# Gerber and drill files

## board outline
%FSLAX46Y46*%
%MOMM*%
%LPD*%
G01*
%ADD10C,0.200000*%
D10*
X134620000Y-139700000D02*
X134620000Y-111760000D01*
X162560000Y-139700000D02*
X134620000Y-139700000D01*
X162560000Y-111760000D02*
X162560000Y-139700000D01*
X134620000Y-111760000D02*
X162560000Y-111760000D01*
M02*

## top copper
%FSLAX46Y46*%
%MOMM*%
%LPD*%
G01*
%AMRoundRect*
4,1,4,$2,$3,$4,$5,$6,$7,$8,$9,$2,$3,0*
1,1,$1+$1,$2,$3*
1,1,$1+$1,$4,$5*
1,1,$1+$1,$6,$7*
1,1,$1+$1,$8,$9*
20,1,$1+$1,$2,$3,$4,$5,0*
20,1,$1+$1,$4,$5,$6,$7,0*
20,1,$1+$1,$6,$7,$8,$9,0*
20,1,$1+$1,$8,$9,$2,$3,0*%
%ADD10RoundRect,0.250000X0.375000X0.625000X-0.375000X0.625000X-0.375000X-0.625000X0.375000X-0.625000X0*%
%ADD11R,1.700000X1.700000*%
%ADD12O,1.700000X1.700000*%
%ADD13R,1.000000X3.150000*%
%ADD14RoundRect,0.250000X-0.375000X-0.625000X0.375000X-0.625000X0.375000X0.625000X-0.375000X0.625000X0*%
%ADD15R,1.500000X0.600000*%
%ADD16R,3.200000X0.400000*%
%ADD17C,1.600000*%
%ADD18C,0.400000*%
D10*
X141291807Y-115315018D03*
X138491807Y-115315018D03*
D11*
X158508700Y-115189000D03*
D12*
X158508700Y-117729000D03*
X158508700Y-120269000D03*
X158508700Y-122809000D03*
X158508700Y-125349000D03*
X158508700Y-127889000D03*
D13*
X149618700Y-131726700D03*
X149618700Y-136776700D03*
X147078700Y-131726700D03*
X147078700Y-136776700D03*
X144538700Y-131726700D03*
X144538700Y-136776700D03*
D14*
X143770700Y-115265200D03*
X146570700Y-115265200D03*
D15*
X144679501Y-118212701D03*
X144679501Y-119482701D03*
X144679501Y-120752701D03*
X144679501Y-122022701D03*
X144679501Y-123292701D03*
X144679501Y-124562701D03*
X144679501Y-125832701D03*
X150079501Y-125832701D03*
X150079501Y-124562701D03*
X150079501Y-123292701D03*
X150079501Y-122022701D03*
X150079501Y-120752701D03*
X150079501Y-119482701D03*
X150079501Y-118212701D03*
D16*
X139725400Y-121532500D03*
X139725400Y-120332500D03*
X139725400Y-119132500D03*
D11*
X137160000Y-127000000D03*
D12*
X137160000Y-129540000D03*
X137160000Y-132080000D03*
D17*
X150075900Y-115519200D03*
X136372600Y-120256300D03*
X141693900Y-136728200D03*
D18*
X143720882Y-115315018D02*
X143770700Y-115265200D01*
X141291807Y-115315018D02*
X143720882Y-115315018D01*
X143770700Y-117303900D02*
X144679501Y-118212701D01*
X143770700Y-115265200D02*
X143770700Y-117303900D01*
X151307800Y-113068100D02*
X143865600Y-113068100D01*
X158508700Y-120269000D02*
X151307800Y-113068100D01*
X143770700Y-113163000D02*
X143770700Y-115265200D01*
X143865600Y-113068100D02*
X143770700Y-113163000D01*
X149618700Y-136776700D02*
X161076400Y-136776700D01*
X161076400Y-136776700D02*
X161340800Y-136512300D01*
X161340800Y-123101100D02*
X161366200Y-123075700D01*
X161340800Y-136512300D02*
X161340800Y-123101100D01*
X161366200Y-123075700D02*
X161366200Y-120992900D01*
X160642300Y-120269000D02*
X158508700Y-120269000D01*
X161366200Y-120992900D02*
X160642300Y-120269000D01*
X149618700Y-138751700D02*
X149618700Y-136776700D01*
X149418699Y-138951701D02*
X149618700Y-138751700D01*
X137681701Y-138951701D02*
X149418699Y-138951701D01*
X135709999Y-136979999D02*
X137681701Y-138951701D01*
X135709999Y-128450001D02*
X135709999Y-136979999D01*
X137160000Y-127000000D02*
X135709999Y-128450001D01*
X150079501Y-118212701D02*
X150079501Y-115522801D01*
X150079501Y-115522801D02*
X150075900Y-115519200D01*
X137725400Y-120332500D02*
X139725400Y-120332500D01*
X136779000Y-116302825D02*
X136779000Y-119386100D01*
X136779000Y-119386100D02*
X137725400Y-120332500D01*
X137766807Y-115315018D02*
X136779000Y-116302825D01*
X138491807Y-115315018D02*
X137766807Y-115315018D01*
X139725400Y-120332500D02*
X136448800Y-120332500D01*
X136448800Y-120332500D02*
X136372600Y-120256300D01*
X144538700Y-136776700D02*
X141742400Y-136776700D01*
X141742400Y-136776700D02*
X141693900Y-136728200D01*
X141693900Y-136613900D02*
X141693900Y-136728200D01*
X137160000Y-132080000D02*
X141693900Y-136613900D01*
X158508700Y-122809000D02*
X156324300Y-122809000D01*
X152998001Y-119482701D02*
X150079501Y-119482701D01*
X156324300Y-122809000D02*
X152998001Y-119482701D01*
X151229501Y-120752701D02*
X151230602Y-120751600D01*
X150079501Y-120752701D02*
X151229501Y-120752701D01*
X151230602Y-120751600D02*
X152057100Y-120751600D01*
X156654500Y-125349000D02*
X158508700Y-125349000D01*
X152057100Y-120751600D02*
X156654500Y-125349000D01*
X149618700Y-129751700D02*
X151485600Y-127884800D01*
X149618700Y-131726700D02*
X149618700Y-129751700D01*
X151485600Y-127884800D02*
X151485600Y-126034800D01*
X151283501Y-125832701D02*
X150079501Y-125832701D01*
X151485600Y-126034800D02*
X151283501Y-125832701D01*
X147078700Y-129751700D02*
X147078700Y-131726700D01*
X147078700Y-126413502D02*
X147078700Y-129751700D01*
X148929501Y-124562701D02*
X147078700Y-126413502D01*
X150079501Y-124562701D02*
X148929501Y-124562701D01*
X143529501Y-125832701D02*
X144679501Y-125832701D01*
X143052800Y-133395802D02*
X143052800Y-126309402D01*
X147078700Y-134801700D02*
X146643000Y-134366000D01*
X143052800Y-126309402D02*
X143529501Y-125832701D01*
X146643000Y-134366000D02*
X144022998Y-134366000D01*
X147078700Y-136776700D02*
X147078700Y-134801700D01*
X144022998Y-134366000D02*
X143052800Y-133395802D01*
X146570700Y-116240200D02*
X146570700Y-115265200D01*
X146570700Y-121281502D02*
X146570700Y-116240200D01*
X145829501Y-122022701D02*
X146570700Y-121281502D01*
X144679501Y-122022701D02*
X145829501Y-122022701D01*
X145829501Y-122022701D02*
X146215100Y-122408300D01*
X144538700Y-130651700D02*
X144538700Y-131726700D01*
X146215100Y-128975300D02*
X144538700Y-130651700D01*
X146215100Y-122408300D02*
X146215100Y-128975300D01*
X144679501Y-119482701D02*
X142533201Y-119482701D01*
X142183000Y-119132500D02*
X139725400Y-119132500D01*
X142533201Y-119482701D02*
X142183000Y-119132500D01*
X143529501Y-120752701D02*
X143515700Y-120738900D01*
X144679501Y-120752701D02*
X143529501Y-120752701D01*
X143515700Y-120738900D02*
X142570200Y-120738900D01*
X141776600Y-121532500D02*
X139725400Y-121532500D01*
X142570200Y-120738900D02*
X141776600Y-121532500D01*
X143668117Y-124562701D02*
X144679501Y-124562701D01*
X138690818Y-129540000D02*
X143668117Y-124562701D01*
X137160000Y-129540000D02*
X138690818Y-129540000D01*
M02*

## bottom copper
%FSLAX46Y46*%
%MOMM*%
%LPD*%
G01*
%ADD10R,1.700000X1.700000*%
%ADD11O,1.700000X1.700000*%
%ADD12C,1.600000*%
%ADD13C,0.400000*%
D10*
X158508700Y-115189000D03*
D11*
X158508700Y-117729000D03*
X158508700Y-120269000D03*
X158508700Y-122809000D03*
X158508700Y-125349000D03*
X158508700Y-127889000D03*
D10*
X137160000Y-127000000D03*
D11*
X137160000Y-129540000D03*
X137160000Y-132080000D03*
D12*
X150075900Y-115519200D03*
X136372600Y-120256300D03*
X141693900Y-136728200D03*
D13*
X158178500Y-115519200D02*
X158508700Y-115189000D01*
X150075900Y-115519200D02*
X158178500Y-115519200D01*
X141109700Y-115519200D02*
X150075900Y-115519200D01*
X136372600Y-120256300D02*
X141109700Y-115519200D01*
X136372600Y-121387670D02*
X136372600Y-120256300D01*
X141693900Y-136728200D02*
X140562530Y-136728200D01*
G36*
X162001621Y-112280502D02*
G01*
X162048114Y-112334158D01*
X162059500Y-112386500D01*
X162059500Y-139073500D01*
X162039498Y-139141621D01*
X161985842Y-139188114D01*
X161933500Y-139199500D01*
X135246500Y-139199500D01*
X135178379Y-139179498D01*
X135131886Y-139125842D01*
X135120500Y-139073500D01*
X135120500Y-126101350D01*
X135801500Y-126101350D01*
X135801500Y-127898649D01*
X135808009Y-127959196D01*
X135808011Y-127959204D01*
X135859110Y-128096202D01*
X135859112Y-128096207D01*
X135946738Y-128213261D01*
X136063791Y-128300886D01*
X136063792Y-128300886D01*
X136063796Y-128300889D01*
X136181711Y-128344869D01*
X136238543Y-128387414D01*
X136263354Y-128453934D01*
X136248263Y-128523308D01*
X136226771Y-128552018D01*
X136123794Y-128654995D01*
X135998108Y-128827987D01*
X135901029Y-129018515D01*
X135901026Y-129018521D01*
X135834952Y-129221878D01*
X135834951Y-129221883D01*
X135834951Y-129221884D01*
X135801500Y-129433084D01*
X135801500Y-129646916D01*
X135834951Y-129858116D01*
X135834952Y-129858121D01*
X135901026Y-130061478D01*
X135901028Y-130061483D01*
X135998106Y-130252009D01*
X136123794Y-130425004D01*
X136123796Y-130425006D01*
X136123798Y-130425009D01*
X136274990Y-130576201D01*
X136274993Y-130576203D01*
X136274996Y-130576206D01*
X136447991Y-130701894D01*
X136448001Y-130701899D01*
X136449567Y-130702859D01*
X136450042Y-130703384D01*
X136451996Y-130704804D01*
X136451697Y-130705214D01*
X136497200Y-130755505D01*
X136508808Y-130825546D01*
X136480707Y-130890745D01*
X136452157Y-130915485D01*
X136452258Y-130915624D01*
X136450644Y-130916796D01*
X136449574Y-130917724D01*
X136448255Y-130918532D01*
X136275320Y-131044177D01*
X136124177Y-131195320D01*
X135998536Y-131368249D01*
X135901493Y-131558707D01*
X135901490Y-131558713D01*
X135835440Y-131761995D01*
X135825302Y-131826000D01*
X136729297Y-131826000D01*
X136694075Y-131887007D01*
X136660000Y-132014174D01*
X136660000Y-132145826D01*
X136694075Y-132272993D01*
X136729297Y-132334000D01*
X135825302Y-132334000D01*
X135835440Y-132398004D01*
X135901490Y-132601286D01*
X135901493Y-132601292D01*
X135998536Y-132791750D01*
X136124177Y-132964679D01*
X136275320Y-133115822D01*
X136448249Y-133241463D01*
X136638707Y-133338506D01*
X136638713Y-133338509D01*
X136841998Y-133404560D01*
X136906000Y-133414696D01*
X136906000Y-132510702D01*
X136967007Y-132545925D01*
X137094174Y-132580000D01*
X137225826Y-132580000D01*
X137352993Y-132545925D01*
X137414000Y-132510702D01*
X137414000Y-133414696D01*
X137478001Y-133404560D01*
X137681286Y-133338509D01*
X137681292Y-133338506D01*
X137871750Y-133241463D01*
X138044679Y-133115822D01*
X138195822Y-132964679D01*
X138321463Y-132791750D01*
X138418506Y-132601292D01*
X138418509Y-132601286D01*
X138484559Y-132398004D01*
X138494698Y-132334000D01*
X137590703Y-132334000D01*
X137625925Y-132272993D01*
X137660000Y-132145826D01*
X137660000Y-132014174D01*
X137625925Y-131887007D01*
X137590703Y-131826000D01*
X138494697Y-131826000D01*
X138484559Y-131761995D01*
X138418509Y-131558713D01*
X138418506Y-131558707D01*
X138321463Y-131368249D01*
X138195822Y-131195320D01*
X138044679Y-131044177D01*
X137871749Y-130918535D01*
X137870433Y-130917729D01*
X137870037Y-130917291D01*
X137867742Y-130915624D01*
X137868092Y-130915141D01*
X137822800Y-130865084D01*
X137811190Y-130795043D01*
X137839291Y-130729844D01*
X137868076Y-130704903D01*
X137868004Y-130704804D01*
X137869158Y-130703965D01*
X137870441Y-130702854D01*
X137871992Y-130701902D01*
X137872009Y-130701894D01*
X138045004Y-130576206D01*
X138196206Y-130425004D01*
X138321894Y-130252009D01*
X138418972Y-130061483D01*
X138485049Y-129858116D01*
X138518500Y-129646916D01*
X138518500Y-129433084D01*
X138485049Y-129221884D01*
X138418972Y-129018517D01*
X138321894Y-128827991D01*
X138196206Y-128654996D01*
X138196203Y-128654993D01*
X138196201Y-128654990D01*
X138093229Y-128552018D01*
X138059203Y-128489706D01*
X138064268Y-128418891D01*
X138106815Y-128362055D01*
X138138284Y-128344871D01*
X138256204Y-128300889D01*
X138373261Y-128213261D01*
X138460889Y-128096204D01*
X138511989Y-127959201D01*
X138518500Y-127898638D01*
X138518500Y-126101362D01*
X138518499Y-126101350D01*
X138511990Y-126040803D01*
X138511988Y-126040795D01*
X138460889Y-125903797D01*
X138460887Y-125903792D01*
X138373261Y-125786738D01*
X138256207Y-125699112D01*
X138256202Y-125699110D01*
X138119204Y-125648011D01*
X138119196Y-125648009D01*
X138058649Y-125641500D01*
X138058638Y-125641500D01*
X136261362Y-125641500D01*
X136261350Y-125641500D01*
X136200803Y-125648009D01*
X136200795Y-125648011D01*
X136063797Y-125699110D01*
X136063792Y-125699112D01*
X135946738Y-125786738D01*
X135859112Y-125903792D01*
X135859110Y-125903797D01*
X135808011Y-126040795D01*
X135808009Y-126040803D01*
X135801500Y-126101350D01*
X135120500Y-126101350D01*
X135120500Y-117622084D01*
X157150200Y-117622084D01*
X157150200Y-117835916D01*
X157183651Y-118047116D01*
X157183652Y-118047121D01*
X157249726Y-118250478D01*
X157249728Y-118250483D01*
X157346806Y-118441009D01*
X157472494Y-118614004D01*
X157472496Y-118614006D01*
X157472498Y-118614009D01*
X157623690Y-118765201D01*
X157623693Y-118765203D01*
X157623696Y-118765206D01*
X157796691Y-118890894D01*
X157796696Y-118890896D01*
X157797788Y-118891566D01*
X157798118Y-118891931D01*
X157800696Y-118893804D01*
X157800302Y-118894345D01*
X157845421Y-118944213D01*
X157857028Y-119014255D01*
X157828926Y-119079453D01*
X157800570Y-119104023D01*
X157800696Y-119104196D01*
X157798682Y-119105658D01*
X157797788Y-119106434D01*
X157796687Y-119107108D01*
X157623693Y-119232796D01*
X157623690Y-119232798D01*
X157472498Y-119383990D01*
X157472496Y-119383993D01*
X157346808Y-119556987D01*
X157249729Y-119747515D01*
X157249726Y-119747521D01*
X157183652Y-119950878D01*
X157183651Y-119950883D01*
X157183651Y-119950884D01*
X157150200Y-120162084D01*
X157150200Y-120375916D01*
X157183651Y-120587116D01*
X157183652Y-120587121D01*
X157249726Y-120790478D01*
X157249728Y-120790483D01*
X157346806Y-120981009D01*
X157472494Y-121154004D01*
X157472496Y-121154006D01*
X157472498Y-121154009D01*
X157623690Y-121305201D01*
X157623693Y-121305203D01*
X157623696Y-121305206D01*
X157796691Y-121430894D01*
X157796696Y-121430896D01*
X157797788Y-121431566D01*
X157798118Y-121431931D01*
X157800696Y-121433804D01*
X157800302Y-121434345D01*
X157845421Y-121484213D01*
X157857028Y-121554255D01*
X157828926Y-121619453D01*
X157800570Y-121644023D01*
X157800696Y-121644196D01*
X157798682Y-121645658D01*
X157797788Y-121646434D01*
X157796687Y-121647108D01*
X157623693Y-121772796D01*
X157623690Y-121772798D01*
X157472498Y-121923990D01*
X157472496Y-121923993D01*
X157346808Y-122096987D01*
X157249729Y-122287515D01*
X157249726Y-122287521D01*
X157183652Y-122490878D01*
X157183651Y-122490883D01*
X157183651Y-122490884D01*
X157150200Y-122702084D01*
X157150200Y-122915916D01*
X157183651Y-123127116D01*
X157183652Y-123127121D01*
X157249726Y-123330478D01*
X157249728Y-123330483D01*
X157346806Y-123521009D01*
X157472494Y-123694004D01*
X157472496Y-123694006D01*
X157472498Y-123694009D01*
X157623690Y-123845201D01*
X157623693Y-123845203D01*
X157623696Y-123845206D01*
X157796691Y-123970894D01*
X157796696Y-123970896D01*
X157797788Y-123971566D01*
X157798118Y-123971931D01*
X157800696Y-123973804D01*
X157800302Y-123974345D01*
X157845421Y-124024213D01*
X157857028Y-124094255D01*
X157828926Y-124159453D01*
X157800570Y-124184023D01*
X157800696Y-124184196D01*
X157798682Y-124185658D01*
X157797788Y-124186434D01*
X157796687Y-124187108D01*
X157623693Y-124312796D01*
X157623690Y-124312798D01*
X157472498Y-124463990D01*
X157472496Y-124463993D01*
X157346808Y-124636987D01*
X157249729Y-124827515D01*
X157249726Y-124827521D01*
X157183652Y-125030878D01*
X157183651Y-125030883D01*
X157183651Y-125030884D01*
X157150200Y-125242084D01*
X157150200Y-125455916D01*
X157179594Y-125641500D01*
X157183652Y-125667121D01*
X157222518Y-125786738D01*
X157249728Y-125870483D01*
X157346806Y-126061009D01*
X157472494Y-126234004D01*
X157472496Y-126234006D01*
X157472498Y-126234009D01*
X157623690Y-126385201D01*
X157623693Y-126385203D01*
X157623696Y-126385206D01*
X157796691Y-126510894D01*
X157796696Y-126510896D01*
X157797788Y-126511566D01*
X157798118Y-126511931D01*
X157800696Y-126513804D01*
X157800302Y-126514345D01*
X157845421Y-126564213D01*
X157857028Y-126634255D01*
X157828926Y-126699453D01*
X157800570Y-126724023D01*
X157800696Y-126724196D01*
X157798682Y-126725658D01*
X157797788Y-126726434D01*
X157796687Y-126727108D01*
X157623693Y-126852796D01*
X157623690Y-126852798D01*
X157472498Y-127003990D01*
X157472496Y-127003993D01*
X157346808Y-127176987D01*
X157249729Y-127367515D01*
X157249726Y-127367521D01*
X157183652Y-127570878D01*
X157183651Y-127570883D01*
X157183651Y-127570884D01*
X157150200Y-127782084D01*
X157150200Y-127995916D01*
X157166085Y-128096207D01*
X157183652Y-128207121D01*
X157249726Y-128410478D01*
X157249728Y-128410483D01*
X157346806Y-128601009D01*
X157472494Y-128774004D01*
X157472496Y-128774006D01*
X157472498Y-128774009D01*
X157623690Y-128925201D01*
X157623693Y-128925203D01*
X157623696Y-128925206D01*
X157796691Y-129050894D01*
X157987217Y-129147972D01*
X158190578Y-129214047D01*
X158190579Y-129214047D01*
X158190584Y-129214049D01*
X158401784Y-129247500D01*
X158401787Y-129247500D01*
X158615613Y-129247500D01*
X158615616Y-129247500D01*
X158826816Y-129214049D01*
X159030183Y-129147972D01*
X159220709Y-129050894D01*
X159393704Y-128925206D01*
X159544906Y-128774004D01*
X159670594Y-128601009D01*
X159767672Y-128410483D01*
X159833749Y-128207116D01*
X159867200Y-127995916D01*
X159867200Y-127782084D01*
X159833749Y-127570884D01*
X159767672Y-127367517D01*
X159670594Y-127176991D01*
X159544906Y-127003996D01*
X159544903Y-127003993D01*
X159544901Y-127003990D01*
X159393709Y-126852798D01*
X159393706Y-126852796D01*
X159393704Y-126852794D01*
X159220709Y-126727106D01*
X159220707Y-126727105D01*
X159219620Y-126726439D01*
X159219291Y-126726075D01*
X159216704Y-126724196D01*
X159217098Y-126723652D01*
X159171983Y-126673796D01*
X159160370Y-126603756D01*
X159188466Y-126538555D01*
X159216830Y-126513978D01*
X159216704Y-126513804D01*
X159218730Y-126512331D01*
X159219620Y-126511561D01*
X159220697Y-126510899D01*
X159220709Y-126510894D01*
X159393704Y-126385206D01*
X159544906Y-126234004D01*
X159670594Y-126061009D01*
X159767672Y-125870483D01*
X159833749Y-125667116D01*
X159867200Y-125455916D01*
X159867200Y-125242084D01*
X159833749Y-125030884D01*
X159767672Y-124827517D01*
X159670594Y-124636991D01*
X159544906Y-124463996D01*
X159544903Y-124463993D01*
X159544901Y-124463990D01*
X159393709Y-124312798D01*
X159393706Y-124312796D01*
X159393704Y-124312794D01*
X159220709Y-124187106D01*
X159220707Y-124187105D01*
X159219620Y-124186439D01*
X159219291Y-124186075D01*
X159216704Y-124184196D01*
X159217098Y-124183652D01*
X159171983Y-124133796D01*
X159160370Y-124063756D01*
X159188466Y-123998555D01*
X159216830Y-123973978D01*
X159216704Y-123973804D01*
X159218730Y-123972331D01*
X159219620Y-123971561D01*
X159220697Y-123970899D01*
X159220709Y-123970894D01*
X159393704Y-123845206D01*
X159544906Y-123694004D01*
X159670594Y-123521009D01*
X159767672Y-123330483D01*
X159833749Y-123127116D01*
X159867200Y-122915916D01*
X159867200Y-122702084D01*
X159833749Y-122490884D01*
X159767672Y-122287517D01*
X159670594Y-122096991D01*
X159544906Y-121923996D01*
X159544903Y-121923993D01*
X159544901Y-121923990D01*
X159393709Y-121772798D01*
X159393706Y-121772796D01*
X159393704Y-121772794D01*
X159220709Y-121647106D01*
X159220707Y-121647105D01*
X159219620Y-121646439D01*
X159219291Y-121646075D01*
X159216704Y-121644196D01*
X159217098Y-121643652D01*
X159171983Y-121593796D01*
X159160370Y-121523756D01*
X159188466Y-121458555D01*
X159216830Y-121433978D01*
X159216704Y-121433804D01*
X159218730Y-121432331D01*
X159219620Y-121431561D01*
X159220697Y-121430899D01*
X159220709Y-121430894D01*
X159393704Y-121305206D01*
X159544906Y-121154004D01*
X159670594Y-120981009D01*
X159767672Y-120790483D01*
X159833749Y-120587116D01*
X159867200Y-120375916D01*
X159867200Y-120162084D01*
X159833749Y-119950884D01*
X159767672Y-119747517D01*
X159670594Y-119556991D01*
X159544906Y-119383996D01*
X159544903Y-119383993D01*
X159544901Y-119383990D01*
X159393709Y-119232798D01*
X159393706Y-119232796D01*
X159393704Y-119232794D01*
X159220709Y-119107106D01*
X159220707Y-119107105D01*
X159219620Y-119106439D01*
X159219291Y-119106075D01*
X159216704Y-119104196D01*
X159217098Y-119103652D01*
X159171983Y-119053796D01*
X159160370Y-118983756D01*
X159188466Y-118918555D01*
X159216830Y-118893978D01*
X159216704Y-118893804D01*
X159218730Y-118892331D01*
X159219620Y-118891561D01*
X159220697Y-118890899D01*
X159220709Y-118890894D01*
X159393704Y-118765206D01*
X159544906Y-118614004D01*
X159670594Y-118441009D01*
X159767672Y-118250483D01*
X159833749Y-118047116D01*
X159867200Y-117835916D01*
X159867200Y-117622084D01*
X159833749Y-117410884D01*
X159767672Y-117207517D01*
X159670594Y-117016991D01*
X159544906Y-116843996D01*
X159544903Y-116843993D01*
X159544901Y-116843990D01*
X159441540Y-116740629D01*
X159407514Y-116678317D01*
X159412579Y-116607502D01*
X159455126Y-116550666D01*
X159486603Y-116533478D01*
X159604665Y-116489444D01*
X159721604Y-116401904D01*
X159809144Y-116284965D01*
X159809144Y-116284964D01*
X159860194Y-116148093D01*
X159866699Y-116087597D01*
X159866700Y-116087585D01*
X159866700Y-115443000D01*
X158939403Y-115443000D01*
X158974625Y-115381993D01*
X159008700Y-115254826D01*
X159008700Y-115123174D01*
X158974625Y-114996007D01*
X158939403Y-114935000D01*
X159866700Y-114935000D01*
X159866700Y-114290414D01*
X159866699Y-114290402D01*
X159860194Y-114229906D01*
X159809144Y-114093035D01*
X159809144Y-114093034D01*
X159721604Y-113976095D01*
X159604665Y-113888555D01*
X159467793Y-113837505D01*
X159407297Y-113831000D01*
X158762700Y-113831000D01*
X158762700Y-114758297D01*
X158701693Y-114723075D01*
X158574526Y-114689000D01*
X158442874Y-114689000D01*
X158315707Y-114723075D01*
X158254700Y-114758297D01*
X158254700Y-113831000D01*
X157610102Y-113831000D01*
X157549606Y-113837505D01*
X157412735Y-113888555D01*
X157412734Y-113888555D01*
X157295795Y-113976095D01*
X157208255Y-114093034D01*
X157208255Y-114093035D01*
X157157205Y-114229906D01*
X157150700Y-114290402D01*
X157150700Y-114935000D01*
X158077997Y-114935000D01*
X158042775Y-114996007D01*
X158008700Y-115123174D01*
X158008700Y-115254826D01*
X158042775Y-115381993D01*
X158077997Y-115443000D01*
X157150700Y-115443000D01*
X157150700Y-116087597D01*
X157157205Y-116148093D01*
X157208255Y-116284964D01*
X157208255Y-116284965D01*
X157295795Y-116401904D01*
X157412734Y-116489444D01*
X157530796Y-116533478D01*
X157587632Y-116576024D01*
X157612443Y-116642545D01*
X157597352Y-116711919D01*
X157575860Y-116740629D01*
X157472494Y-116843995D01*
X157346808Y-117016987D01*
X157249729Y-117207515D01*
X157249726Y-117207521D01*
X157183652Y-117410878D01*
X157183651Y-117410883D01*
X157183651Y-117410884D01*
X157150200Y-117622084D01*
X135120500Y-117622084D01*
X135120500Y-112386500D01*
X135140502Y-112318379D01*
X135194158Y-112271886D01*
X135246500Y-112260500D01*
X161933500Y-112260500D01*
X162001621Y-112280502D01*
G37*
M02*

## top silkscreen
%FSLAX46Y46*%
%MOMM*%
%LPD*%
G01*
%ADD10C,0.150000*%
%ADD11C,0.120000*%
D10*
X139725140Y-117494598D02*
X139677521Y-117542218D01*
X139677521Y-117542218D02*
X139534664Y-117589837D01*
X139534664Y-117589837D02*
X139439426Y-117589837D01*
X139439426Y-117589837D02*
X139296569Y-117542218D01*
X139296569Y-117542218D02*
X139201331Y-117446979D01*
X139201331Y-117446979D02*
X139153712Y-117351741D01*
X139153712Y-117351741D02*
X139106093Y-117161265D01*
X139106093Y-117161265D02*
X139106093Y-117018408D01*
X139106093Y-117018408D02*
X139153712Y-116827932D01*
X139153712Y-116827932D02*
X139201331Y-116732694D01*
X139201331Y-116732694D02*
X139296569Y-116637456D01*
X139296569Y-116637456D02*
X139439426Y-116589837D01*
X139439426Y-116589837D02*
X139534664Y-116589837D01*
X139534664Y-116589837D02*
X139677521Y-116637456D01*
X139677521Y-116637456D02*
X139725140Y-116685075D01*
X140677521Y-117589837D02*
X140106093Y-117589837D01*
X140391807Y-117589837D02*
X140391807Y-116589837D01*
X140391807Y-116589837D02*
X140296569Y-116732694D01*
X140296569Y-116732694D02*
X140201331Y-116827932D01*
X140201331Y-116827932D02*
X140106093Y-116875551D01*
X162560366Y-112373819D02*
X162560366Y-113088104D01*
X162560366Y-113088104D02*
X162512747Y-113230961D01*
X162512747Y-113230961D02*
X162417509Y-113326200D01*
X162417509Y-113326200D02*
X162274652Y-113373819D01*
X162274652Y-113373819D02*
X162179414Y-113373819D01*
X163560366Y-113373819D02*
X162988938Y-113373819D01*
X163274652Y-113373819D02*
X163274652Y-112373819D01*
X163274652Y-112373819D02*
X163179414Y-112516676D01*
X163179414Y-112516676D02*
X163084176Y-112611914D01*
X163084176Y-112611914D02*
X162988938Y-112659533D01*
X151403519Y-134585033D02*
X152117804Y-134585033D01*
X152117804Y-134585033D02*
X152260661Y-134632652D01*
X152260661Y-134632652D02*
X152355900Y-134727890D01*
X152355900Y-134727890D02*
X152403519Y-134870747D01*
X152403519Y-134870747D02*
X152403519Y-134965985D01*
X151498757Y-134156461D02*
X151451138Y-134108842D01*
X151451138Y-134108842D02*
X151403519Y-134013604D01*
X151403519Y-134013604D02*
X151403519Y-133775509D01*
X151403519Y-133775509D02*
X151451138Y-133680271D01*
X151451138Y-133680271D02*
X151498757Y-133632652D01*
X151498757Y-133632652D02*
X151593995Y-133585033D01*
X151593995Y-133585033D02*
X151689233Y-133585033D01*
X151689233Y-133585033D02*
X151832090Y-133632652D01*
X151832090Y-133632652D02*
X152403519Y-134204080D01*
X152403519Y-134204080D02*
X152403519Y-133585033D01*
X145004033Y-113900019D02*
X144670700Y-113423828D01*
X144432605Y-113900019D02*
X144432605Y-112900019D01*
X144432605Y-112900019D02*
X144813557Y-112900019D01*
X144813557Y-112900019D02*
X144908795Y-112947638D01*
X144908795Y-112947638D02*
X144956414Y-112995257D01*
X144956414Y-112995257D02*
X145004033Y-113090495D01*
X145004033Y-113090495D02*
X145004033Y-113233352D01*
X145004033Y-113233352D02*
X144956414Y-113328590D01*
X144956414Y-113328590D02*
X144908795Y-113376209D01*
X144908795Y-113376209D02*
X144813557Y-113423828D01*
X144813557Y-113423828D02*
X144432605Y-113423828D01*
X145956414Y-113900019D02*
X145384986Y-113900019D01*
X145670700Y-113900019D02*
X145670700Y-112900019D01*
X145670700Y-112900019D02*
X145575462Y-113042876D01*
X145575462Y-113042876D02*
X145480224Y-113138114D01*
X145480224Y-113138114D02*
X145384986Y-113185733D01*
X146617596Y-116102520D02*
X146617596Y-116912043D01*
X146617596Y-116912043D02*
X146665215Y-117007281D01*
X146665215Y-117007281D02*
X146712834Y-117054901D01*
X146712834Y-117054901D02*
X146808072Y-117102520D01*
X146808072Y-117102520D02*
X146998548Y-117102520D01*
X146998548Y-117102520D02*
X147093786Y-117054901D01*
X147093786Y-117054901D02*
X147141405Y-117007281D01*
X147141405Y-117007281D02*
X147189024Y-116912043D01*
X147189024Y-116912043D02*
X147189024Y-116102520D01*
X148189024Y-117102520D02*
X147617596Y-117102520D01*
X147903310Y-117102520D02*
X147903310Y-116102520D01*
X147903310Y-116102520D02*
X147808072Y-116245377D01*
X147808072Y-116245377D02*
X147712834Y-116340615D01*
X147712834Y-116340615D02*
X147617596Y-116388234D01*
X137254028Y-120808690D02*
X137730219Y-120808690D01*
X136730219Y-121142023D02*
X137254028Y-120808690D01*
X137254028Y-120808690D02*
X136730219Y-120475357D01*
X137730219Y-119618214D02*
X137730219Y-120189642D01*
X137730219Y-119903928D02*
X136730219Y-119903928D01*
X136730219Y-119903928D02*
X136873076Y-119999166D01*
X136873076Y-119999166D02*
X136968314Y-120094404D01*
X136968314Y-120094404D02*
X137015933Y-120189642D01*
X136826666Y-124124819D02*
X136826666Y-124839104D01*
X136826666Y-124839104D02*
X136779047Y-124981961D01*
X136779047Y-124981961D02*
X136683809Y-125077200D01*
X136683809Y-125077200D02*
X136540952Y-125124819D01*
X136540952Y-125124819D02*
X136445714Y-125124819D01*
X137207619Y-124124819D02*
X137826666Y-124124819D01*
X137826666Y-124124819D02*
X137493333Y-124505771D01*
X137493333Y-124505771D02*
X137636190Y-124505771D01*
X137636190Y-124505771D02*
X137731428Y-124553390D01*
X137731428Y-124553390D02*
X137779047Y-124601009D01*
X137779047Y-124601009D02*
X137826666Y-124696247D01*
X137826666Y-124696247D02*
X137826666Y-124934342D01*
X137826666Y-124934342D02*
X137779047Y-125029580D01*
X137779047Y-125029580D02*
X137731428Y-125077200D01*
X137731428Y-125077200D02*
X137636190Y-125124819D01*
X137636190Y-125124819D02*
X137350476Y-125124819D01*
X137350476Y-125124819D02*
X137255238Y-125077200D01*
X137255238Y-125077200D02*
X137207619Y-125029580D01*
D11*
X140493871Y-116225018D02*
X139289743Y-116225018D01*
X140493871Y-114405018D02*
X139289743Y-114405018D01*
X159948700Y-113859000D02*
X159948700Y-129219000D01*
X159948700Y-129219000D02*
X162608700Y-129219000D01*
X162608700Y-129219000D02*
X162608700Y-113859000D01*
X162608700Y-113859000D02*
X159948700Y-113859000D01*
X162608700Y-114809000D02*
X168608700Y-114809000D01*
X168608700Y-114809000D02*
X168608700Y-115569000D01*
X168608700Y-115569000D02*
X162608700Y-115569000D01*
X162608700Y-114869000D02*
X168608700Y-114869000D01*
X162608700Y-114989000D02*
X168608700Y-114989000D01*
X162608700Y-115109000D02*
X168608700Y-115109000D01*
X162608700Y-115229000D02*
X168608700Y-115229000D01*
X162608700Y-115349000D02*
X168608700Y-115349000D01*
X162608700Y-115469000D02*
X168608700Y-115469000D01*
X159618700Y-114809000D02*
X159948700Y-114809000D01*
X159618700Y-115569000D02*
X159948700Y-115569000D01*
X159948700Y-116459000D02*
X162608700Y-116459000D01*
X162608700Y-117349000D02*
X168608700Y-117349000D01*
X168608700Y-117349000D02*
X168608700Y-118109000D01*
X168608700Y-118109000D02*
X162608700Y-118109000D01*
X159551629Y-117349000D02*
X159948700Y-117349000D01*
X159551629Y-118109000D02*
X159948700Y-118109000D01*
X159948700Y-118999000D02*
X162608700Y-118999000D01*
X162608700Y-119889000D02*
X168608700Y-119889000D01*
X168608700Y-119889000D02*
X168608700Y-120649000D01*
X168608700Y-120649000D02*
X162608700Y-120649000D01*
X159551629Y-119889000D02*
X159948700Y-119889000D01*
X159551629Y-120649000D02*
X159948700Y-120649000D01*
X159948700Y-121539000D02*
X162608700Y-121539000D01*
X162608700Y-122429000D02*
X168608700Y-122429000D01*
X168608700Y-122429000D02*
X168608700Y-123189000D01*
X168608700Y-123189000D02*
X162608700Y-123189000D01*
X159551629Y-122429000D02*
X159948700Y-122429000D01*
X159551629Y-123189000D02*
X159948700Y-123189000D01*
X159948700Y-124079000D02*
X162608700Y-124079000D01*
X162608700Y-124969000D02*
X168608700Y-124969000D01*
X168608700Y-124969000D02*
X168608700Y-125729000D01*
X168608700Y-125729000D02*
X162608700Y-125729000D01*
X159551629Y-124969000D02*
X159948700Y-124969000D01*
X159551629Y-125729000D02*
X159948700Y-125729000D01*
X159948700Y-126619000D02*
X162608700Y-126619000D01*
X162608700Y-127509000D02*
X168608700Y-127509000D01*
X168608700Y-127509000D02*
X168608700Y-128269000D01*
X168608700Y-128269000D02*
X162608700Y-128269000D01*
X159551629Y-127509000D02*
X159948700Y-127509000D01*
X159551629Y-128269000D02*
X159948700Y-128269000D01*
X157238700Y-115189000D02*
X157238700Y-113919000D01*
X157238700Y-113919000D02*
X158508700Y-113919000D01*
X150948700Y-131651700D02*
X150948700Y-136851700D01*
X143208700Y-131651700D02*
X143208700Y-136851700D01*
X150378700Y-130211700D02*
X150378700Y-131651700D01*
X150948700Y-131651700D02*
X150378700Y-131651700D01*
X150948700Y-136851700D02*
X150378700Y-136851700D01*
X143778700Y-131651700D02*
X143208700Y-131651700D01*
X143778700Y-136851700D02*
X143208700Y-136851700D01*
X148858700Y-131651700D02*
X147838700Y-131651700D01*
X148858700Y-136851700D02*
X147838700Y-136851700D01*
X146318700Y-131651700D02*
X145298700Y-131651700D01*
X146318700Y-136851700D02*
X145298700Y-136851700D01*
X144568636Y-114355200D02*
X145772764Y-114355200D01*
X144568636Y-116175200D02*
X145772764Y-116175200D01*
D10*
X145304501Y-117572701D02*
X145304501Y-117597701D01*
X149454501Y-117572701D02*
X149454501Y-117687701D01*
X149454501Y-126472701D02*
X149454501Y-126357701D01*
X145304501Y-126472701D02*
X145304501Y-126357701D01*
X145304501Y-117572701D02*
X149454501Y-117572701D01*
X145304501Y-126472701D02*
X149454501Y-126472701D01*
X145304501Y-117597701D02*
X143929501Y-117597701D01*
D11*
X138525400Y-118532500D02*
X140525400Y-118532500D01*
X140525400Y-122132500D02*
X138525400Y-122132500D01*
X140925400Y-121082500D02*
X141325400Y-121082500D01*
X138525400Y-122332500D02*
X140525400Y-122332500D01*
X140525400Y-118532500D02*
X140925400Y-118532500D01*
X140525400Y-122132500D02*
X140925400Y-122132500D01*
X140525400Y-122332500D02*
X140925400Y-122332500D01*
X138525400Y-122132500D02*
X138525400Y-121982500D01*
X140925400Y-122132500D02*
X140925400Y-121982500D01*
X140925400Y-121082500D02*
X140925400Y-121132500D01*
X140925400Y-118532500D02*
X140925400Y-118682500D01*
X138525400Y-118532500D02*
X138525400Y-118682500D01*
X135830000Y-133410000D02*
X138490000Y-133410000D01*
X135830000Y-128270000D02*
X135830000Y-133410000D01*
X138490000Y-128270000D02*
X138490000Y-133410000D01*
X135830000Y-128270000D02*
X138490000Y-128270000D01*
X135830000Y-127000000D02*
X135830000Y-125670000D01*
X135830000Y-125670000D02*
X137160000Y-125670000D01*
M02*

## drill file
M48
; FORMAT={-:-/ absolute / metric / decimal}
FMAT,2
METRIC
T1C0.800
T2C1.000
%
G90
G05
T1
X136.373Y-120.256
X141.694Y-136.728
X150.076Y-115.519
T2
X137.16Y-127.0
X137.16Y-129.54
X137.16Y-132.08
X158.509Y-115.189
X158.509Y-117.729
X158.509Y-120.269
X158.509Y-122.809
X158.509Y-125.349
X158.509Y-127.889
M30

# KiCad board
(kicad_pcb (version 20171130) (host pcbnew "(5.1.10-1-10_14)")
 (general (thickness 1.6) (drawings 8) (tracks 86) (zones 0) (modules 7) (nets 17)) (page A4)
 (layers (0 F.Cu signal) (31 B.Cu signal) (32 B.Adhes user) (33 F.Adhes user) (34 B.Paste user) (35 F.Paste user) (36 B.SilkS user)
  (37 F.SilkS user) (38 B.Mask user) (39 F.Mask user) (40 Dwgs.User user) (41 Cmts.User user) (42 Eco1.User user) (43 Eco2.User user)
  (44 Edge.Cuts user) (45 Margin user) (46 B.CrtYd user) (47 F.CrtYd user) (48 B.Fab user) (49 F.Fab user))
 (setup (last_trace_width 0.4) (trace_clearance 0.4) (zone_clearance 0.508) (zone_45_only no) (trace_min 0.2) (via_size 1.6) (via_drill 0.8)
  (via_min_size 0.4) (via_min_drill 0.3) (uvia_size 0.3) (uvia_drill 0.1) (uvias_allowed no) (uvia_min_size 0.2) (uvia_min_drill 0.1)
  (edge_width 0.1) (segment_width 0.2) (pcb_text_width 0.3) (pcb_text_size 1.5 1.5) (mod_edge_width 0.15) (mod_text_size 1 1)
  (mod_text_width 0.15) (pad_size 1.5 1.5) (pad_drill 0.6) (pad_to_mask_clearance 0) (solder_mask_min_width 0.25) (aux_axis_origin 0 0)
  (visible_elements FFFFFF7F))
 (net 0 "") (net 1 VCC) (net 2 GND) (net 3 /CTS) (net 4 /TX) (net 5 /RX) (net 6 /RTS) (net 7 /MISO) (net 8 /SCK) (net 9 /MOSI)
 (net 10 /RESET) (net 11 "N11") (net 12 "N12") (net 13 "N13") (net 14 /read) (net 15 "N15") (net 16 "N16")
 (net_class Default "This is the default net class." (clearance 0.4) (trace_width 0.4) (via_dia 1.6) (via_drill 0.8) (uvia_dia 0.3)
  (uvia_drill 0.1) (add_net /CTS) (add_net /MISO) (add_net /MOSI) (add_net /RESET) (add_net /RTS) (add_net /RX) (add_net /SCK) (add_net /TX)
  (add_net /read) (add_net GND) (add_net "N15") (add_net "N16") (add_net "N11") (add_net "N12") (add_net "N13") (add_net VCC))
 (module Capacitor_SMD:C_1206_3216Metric (layer F.Cu) (at 139.891807 115.315018 180)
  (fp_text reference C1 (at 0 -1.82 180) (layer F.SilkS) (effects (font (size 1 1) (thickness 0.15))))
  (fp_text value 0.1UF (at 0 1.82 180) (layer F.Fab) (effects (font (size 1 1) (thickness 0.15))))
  (fp_line (start -0.602064 -0.91) (end 0.602064 -0.91) (layer F.SilkS) (width 0.12))
  (fp_line (start -0.602064 0.91) (end 0.602064 0.91) (layer F.SilkS) (width 0.12))
  (pad 1 smd roundrect (at -1.4 0 180) (size 1.25 1.75) (layers F.Cu F.Paste F.Mask) (roundrect_rratio 0.2) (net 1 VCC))
  (pad 2 smd roundrect (at 1.4 0 180) (size 1.25 1.75) (layers F.Cu F.Paste F.Mask) (roundrect_rratio 0.2) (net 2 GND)))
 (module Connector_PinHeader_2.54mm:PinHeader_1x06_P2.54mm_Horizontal (layer F.Cu) (at 158.5087 115.189)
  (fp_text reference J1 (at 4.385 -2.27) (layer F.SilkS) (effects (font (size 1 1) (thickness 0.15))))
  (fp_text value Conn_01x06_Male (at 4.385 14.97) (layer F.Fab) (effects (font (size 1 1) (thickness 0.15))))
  (fp_line (start 1.44 -1.33) (end 1.44 14.03) (layer F.SilkS) (width 0.12))
  (fp_line (start 1.44 14.03) (end 4.1 14.03) (layer F.SilkS) (width 0.12))
  (fp_line (start 4.1 14.03) (end 4.1 -1.33) (layer F.SilkS) (width 0.12))
  (fp_line (start 4.1 -1.33) (end 1.44 -1.33) (layer F.SilkS) (width 0.12))
  (fp_line (start 4.1 -0.38) (end 10.1 -0.38) (layer F.SilkS) (width 0.12))
  (fp_line (start 10.1 -0.38) (end 10.1 0.38) (layer F.SilkS) (width 0.12))
  (fp_line (start 10.1 0.38) (end 4.1 0.38) (layer F.SilkS) (width 0.12))
  (fp_line (start 4.1 -0.32) (end 10.1 -0.32) (layer F.SilkS) (width 0.12))
  (fp_line (start 4.1 -0.2) (end 10.1 -0.2) (layer F.SilkS) (width 0.12))
  (fp_line (start 4.1 -0.08) (end 10.1 -0.08) (layer F.SilkS) (width 0.12))
  (fp_line (start 4.1 0.04) (end 10.1 0.04) (layer F.SilkS) (width 0.12))
  (fp_line (start 4.1 0.16) (end 10.1 0.16) (layer F.SilkS) (width 0.12))
  (fp_line (start 4.1 0.28) (end 10.1 0.28) (layer F.SilkS) (width 0.12))
  (fp_line (start 1.11 -0.38) (end 1.44 -0.38) (layer F.SilkS) (width 0.12))
  (fp_line (start 1.11 0.38) (end 1.44 0.38) (layer F.SilkS) (width 0.12))
  (fp_line (start 1.44 1.27) (end 4.1 1.27) (layer F.SilkS) (width 0.12))
  (fp_line (start 4.1 2.16) (end 10.1 2.16) (layer F.SilkS) (width 0.12))
  (fp_line (start 10.1 2.16) (end 10.1 2.92) (layer F.SilkS) (width 0.12))
  (fp_line (start 10.1 2.92) (end 4.1 2.92) (layer F.SilkS) (width 0.12))
  (fp_line (start 1.042929 2.16) (end 1.44 2.16) (layer F.SilkS) (width 0.12))
  (fp_line (start 1.042929 2.92) (end 1.44 2.92) (layer F.SilkS) (width 0.12))
  (fp_line (start 1.44 3.81) (end 4.1 3.81) (layer F.SilkS) (width 0.12))
  (fp_line (start 4.1 4.7) (end 10.1 4.7) (layer F.SilkS) (width 0.12))
  (fp_line (start 10.1 4.7) (end 10.1 5.46) (layer F.SilkS) (width 0.12))
  (fp_line (start 10.1 5.46) (end 4.1 5.46) (layer F.SilkS) (width 0.12))
  (fp_line (start 1.042929 4.7) (end 1.44 4.7) (layer F.SilkS) (width 0.12))
  (fp_line (start 1.042929 5.46) (end 1.44 5.46) (layer F.SilkS) (width 0.12))
  (fp_line (start 1.44 6.35) (end 4.1 6.35) (layer F.SilkS) (width 0.12))
  (fp_line (start 4.1 7.24) (end 10.1 7.24) (layer F.SilkS) (width 0.12))
  (fp_line (start 10.1 7.24) (end 10.1 8) (layer F.SilkS) (width 0.12))
  (fp_line (start 10.1 8) (end 4.1 8) (layer F.SilkS) (width 0.12))
  (fp_line (start 1.042929 7.24) (end 1.44 7.24) (layer F.SilkS) (width 0.12))
  (fp_line (start 1.042929 8) (end 1.44 8) (layer F.SilkS) (width 0.12))
  (fp_line (start 1.44 8.89) (end 4.1 8.89) (layer F.SilkS) (width 0.12))
  (fp_line (start 4.1 9.78) (end 10.1 9.78) (layer F.SilkS) (width 0.12))
  (fp_line (start 10.1 9.78) (end 10.1 10.54) (layer F.SilkS) (width 0.12))
  (fp_line (start 10.1 10.54) (end 4.1 10.54) (layer F.SilkS) (width 0.12))
  (fp_line (start 1.042929 9.78) (end 1.44 9.78) (layer F.SilkS) (width 0.12))
  (fp_line (start 1.042929 10.54) (end 1.44 10.54) (layer F.SilkS) (width 0.12))
  (fp_line (start 1.44 11.43) (end 4.1 11.43) (layer F.SilkS) (width 0.12))
  (fp_line (start 4.1 12.32) (end 10.1 12.32) (layer F.SilkS) (width 0.12))
  (fp_line (start 10.1 12.32) (end 10.1 13.08) (layer F.SilkS) (width 0.12))
  (fp_line (start 10.1 13.08) (end 4.1 13.08) (layer F.SilkS) (width 0.12))
  (fp_line (start 1.042929 12.32) (end 1.44 12.32) (layer F.SilkS) (width 0.12))
  (fp_line (start 1.042929 13.08) (end 1.44 13.08) (layer F.SilkS) (width 0.12))
  (fp_line (start -1.27 0) (end -1.27 -1.27) (layer F.SilkS) (width 0.12))
  (fp_line (start -1.27 -1.27) (end 0 -1.27) (layer F.SilkS) (width 0.12))
  (pad 1 thru_hole rect (at 0 0) (size 1.7 1.7) (drill 1) (layers *.Cu *.Mask) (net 2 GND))
  (pad 2 thru_hole oval (at 0 2.54) (size 1.7 1.7) (drill 1) (layers *.Cu *.Mask) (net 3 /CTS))
  (pad 3 thru_hole oval (at 0 5.08) (size 1.7 1.7) (drill 1) (layers *.Cu *.Mask) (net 1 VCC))
  (pad 4 thru_hole oval (at 0 7.62) (size 1.7 1.7) (drill 1) (layers *.Cu *.Mask) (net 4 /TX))
  (pad 5 thru_hole oval (at 0 10.16) (size 1.7 1.7) (drill 1) (layers *.Cu *.Mask) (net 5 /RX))
  (pad 6 thru_hole oval (at 0 12.7) (size 1.7 1.7) (drill 1) (layers *.Cu *.Mask) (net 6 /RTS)))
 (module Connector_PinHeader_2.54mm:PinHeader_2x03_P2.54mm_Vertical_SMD (layer F.Cu) (at 147.0787 134.2517 270)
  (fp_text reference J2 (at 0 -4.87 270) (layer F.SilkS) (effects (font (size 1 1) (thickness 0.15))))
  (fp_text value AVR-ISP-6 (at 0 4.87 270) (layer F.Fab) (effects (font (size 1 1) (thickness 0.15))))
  (fp_line (start -2.6 -3.87) (end 2.6 -3.87) (layer F.SilkS) (width 0.12))
  (fp_line (start -2.6 3.87) (end 2.6 3.87) (layer F.SilkS) (width 0.12))
  (fp_line (start -4.04 -3.3) (end -2.6 -3.3) (layer F.SilkS) (width 0.12))
  (fp_line (start -2.6 -3.87) (end -2.6 -3.3) (layer F.SilkS) (width 0.12))
  (fp_line (start 2.6 -3.87) (end 2.6 -3.3) (layer F.SilkS) (width 0.12))
  (fp_line (start -2.6 3.3) (end -2.6 3.87) (layer F.SilkS) (width 0.12))
  (fp_line (start 2.6 3.3) (end 2.6 3.87) (layer F.SilkS) (width 0.12))
  (fp_line (start -2.6 -1.78) (end -2.6 -0.76) (layer F.SilkS) (width 0.12))
  (fp_line (start 2.6 -1.78) (end 2.6 -0.76) (layer F.SilkS) (width 0.12))
  (fp_line (start -2.6 0.76) (end -2.6 1.78) (layer F.SilkS) (width 0.12))
  (fp_line (start 2.6 0.76) (end 2.6 1.78) (layer F.SilkS) (width 0.12))
  (pad 1 smd rect (at -2.525 -2.54 270) (size 3.15 1) (layers F.Cu F.Paste F.Mask) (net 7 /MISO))
  (pad 2 smd rect (at 2.525 -2.54 270) (size 3.15 1) (layers F.Cu F.Paste F.Mask) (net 1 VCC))
  (pad 3 smd rect (at -2.525 0 270) (size 3.15 1) (layers F.Cu F.Paste F.Mask) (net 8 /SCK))
  (pad 4 smd rect (at 2.525 0 270) (size 3.15 1) (layers F.Cu F.Paste F.Mask) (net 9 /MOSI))
  (pad 5 smd rect (at -2.525 2.54 270) (size 3.15 1) (layers F.Cu F.Paste F.Mask) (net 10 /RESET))
  (pad 6 smd rect (at 2.525 2.54 270) (size 3.15 1) (layers F.Cu F.Paste F.Mask) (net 2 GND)))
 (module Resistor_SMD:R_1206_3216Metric (layer F.Cu) (at 145.1707 115.2652)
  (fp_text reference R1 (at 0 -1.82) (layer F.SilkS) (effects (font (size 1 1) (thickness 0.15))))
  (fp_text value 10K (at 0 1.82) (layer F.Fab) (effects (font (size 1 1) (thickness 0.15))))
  (fp_line (start -0.602064 -0.91) (end 0.602064 -0.91) (layer F.SilkS) (width 0.12))
  (fp_line (start -0.602064 0.91) (end 0.602064 0.91) (layer F.SilkS) (width 0.12))
  (pad 1 smd roundrect (at -1.4 0) (size 1.25 1.75) (layers F.Cu F.Paste F.Mask) (roundrect_rratio 0.2) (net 1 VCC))
  (pad 2 smd roundrect (at 1.4 0) (size 1.25 1.75) (layers F.Cu F.Paste F.Mask) (roundrect_rratio 0.2) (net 10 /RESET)))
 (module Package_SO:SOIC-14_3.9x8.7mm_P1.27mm (layer F.Cu) (at 147.379501 122.022701)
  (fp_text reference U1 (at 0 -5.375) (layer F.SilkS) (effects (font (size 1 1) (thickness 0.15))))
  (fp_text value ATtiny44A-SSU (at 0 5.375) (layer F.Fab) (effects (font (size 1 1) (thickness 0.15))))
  (fp_line (start -2.075 -4.45) (end -2.075 -4.425) (layer F.SilkS) (width 0.15))
  (fp_line (start 2.075 -4.45) (end 2.075 -4.335) (layer F.SilkS) (width 0.15))
  (fp_line (start 2.075 4.45) (end 2.075 4.335) (layer F.SilkS) (width 0.15))
  (fp_line (start -2.075 4.45) (end -2.075 4.335) (layer F.SilkS) (width 0.15))
  (fp_line (start -2.075 -4.45) (end 2.075 -4.45) (layer F.SilkS) (width 0.15))
  (fp_line (start -2.075 4.45) (end 2.075 4.45) (layer F.SilkS) (width 0.15))
  (fp_line (start -2.075 -4.425) (end -3.45 -4.425) (layer F.SilkS) (width 0.15))
  (pad 1 smd rect (at -2.7 -3.81) (size 1.5 0.6) (layers F.Cu F.Paste F.Mask) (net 1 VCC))
  (pad 2 smd rect (at -2.7 -2.54) (size 1.5 0.6) (layers F.Cu F.Paste F.Mask) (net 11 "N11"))
  (pad 3 smd rect (at -2.7 -1.27) (size 1.5 0.6) (layers F.Cu F.Paste F.Mask) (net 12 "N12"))
  (pad 4 smd rect (at -2.7 0) (size 1.5 0.6) (layers F.Cu F.Paste F.Mask) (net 10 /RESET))
  (pad 5 smd rect (at -2.7 1.27) (size 1.5 0.6) (layers F.Cu F.Paste F.Mask) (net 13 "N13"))
  (pad 6 smd rect (at -2.7 2.54) (size 1.5 0.6) (layers F.Cu F.Paste F.Mask) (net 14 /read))
  (pad 7 smd rect (at -2.7 3.81) (size 1.5 0.6) (layers F.Cu F.Paste F.Mask) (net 9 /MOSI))
  (pad 8 smd rect (at 2.7 3.81) (size 1.5 0.6) (layers F.Cu F.Paste F.Mask) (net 7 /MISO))
  (pad 9 smd rect (at 2.7 2.54) (size 1.5 0.6) (layers F.Cu F.Paste F.Mask) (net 8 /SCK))
  (pad 10 smd rect (at 2.7 1.27) (size 1.5 0.6) (layers F.Cu F.Paste F.Mask) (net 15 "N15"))
  (pad 11 smd rect (at 2.7 0) (size 1.5 0.6) (layers F.Cu F.Paste F.Mask) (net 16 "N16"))
  (pad 12 smd rect (at 2.7 -1.27) (size 1.5 0.6) (layers F.Cu F.Paste F.Mask) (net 5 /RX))
  (pad 13 smd rect (at 2.7 -2.54) (size 1.5 0.6) (layers F.Cu F.Paste F.Mask) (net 4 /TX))
  (pad 14 smd rect (at 2.7 -3.81) (size 1.5 0.6) (layers F.Cu F.Paste F.Mask) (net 2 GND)))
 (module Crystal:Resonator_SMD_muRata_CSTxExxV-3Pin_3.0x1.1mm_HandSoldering (layer F.Cu) (at 139.7254 120.3325 90)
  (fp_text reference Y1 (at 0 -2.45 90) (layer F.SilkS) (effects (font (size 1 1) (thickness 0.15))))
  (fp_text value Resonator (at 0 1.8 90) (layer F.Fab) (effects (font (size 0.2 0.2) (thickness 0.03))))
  (fp_line (start 1.8 -1.2) (end 1.8 0.8) (layer F.SilkS) (width 0.12))
  (fp_line (start -1.8 0.8) (end -1.8 -1.2) (layer F.SilkS) (width 0.12))
  (fp_line (start -0.75 1.2) (end -0.75 1.6) (layer F.SilkS) (width 0.12))
  (fp_line (start -2 -1.2) (end -2 0.8) (layer F.SilkS) (width 0.12))
  (fp_line (start 1.8 0.8) (end 1.8 1.2) (layer F.SilkS) (width 0.12))
  (fp_line (start -1.8 0.8) (end -1.8 1.2) (layer F.SilkS) (width 0.12))
  (fp_line (start -2 0.8) (end -2 1.2) (layer F.SilkS) (width 0.12))
  (fp_line (start -1.8 -1.2) (end -1.65 -1.2) (layer F.SilkS) (width 0.12))
  (fp_line (start -1.8 1.2) (end -1.65 1.2) (layer F.SilkS) (width 0.12))
  (fp_line (start -0.75 1.2) (end -0.8 1.2) (layer F.SilkS) (width 0.12))
  (fp_line (start 1.8 1.2) (end 1.65 1.2) (layer F.SilkS) (width 0.12))
  (fp_line (start 1.8 -1.2) (end 1.65 -1.2) (layer F.SilkS) (width 0.12))
  (pad 1 smd rect (at -1.2 0 90) (size 0.4 3.2) (layers F.Cu F.Paste F.Mask) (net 12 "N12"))
  (pad 2 smd rect (at 0 0 90) (size 0.4 3.2) (layers F.Cu F.Paste F.Mask) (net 2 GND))
  (pad 3 smd rect (at 1.2 0 90) (size 0.4 3.2) (layers F.Cu F.Paste F.Mask) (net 11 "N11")))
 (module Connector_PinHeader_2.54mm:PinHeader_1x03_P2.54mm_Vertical (layer F.Cu) (at 137.16 127)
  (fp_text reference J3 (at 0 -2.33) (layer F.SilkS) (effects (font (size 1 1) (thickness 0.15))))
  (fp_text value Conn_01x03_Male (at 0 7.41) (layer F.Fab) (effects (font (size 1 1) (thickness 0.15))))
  (fp_line (start -1.33 6.41) (end 1.33 6.41) (layer F.SilkS) (width 0.12))
  (fp_line (start -1.33 1.27) (end -1.33 6.41) (layer F.SilkS) (width 0.12))
  (fp_line (start 1.33 1.27) (end 1.33 6.41) (layer F.SilkS) (width 0.12))
  (fp_line (start -1.33 1.27) (end 1.33 1.27) (layer F.SilkS) (width 0.12))
  (fp_line (start -1.33 0) (end -1.33 -1.33) (layer F.SilkS) (width 0.12))
  (fp_line (start -1.33 -1.33) (end 0 -1.33) (layer F.SilkS) (width 0.12))
  (pad 1 thru_hole rect (at 0 0) (size 1.7 1.7) (drill 1) (layers *.Cu *.Mask) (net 1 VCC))
  (pad 2 thru_hole oval (at 0 2.54) (size 1.7 1.7) (drill 1) (layers *.Cu *.Mask) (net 14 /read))
  (pad 3 thru_hole oval (at 0 5.08) (size 1.7 1.7) (drill 1) (layers *.Cu *.Mask) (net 2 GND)))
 (gr_line (start 134.62 139.7) (end 134.62 111.76) (layer Edge.Cuts) (width 0.2))
 (gr_line (start 162.56 139.7) (end 134.62 139.7) (layer Edge.Cuts) (width 0.2))
 (gr_line (start 162.56 111.76) (end 162.56 139.7) (layer Edge.Cuts) (width 0.2))
 (gr_line (start 134.62 111.76) (end 162.56 111.76) (layer Edge.Cuts) (width 0.2))
 (segment (start 143.720882 115.315018) (end 143.7707 115.2652) (width 0.4) (layer F.Cu) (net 1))
 (segment (start 141.291807 115.315018) (end 143.720882 115.315018) (width 0.4) (layer F.Cu) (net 1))
 (segment (start 143.7707 117.3039) (end 144.679501 118.212701) (width 0.4) (layer F.Cu) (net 1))
 (segment (start 143.7707 115.2652) (end 143.7707 117.3039) (width 0.4) (layer F.Cu) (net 1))
 (segment (start 151.3078 113.0681) (end 143.8656 113.0681) (width 0.4) (layer F.Cu) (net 1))
 (segment (start 158.5087 120.269) (end 151.3078 113.0681) (width 0.4) (layer F.Cu) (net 1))
 (segment (start 143.7707 113.163) (end 143.7707 115.2652) (width 0.4) (layer F.Cu) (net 1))
 (segment (start 143.8656 113.0681) (end 143.7707 113.163) (width 0.4) (layer F.Cu) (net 1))
 (segment (start 149.6187 136.7767) (end 161.0764 136.7767) (width 0.4) (layer F.Cu) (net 1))
 (segment (start 161.0764 136.7767) (end 161.3408 136.5123) (width 0.4) (layer F.Cu) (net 1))
 (segment (start 161.3408 123.1011) (end 161.3662 123.0757) (width 0.4) (layer F.Cu) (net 1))
 (segment (start 161.3408 136.5123) (end 161.3408 123.1011) (width 0.4) (layer F.Cu) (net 1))
 (segment (start 161.3662 123.0757) (end 161.3662 120.9929) (width 0.4) (layer F.Cu) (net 1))
 (segment (start 160.6423 120.269) (end 158.5087 120.269) (width 0.4) (layer F.Cu) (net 1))
 (segment (start 161.3662 120.9929) (end 160.6423 120.269) (width 0.4) (layer F.Cu) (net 1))
 (segment (start 149.6187 138.7517) (end 149.6187 136.7767) (width 0.4) (layer F.Cu) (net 1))
 (segment (start 149.418699 138.951701) (end 149.6187 138.7517) (width 0.4) (layer F.Cu) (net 1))
 (segment (start 137.681701 138.951701) (end 149.418699 138.951701) (width 0.4) (layer F.Cu) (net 1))
 (segment (start 135.709999 136.979999) (end 137.681701 138.951701) (width 0.4) (layer F.Cu) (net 1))
 (segment (start 135.709999 128.450001) (end 135.709999 136.979999) (width 0.4) (layer F.Cu) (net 1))
 (segment (start 137.16 127) (end 135.709999 128.450001) (width 0.4) (layer F.Cu) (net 1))
 (via (at 150.0759 115.5192) (size 1.6) (drill 0.8) (layers F.Cu B.Cu) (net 2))
 (segment (start 150.079501 118.212701) (end 150.079501 115.522801) (width 0.4) (layer F.Cu) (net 2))
 (segment (start 150.079501 115.522801) (end 150.0759 115.5192) (width 0.4) (layer F.Cu) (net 2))
 (segment (start 158.1785 115.5192) (end 158.5087 115.189) (width 0.4) (layer B.Cu) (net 2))
 (segment (start 150.0759 115.5192) (end 158.1785 115.5192) (width 0.4) (layer B.Cu) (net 2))
 (segment (start 137.7254 120.3325) (end 139.7254 120.3325) (width 0.4) (layer F.Cu) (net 2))
 (segment (start 136.779 116.302825) (end 136.779 119.3861) (width 0.4) (layer F.Cu) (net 2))
 (segment (start 136.779 119.3861) (end 137.7254 120.3325) (width 0.4) (layer F.Cu) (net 2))
 (segment (start 137.766807 115.315018) (end 136.779 116.302825) (width 0.4) (layer F.Cu) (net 2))
 (segment (start 138.491807 115.315018) (end 137.766807 115.315018) (width 0.4) (layer F.Cu) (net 2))
 (via (at 136.3726 120.2563) (size 1.6) (drill 0.8) (layers F.Cu B.Cu) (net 2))
 (segment (start 139.7254 120.3325) (end 136.4488 120.3325) (width 0.4) (layer F.Cu) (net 2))
 (segment (start 136.4488 120.3325) (end 136.3726 120.2563) (width 0.4) (layer F.Cu) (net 2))
 (segment (start 141.1097 115.5192) (end 150.0759 115.5192) (width 0.4) (layer B.Cu) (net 2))
 (segment (start 136.3726 120.2563) (end 141.1097 115.5192) (width 0.4) (layer B.Cu) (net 2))
 (via (at 141.6939 136.7282) (size 1.6) (drill 0.8) (layers F.Cu B.Cu) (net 2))
 (segment (start 144.5387 136.7767) (end 141.7424 136.7767) (width 0.4) (layer F.Cu) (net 2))
 (segment (start 141.7424 136.7767) (end 141.6939 136.7282) (width 0.4) (layer F.Cu) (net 2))
 (segment (start 136.3726 121.38767) (end 136.3726 120.2563) (width 0.4) (layer B.Cu) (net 2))
 (segment (start 141.6939 136.7282) (end 140.56253 136.7282) (width 0.4) (layer B.Cu) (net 2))
 (segment (start 141.6939 136.6139) (end 141.6939 136.7282) (width 0.4) (layer F.Cu) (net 2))
 (segment (start 137.16 132.08) (end 141.6939 136.6139) (width 0.4) (layer F.Cu) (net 2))
 (segment (start 158.5087 122.809) (end 156.3243 122.809) (width 0.4) (layer F.Cu) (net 4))
 (segment (start 152.998001 119.482701) (end 150.079501 119.482701) (width 0.4) (layer F.Cu) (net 4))
 (segment (start 156.3243 122.809) (end 152.998001 119.482701) (width 0.4) (layer F.Cu) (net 4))
 (segment (start 151.229501 120.752701) (end 151.230602 120.7516) (width 0.4) (layer F.Cu) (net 5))
 (segment (start 150.079501 120.752701) (end 151.229501 120.752701) (width 0.4) (layer F.Cu) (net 5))
 (segment (start 151.230602 120.7516) (end 152.0571 120.7516) (width 0.4) (layer F.Cu) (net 5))
 (segment (start 156.6545 125.349) (end 158.5087 125.349) (width 0.4) (layer F.Cu) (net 5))
 (segment (start 152.0571 120.7516) (end 156.6545 125.349) (width 0.4) (layer F.Cu) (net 5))
 (segment (start 149.6187 129.7517) (end 151.4856 127.8848) (width 0.4) (layer F.Cu) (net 7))
 (segment (start 149.6187 131.7267) (end 149.6187 129.7517) (width 0.4) (layer F.Cu) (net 7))
 (segment (start 151.4856 127.8848) (end 151.4856 126.0348) (width 0.4) (layer F.Cu) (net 7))
 (segment (start 151.283501 125.832701) (end 150.079501 125.832701) (width 0.4) (layer F.Cu) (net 7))
 (segment (start 151.4856 126.0348) (end 151.283501 125.832701) (width 0.4) (layer F.Cu) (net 7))
 (segment (start 147.0787 129.7517) (end 147.0787 131.7267) (width 0.4) (layer F.Cu) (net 8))
 (segment (start 147.0787 126.413502) (end 147.0787 129.7517) (width 0.4) (layer F.Cu) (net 8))
 (segment (start 148.929501 124.562701) (end 147.0787 126.413502) (width 0.4) (layer F.Cu) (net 8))
 (segment (start 150.079501 124.562701) (end 148.929501 124.562701) (width 0.4) (layer F.Cu) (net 8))
 (segment (start 143.529501 125.832701) (end 144.679501 125.832701) (width 0.4) (layer F.Cu) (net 9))
 (segment (start 143.0528 133.395802) (end 143.0528 126.309402) (width 0.4) (layer F.Cu) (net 9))
 (segment (start 147.0787 134.8017) (end 146.643 134.366) (width 0.4) (layer F.Cu) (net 9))
 (segment (start 143.0528 126.309402) (end 143.529501 125.832701) (width 0.4) (layer F.Cu) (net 9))
 (segment (start 146.643 134.366) (end 144.022998 134.366) (width 0.4) (layer F.Cu) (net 9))
 (segment (start 147.0787 136.7767) (end 147.0787 134.8017) (width 0.4) (layer F.Cu) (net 9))
 (segment (start 144.022998 134.366) (end 143.0528 133.395802) (width 0.4) (layer F.Cu) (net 9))
 (segment (start 146.5707 116.2402) (end 146.5707 115.2652) (width 0.4) (layer F.Cu) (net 10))
 (segment (start 146.5707 121.281502) (end 146.5707 116.2402) (width 0.4) (layer F.Cu) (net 10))
 (segment (start 145.829501 122.022701) (end 146.5707 121.281502) (width 0.4) (layer F.Cu) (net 10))
 (segment (start 144.679501 122.022701) (end 145.829501 122.022701) (width 0.4) (layer F.Cu) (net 10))
 (segment (start 145.829501 122.022701) (end 146.2151 122.4083) (width 0.4) (layer F.Cu) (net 10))
 (segment (start 144.5387 130.6517) (end 144.5387 131.7267) (width 0.4) (layer F.Cu) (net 10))
 (segment (start 146.2151 128.9753) (end 144.5387 130.6517) (width 0.4) (layer F.Cu) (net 10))
 (segment (start 146.2151 122.4083) (end 146.2151 128.9753) (width 0.4) (layer F.Cu) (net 10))
 (segment (start 144.679501 119.482701) (end 142.533201 119.482701) (width 0.4) (layer F.Cu) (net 11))
 (segment (start 142.183 119.1325) (end 139.7254 119.1325) (width 0.4) (layer F.Cu) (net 11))
 (segment (start 142.533201 119.482701) (end 142.183 119.1325) (width 0.4) (layer F.Cu) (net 11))
 (segment (start 143.529501 120.752701) (end 143.5157 120.7389) (width 0.4) (layer F.Cu) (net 12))
 (segment (start 144.679501 120.752701) (end 143.529501 120.752701) (width 0.4) (layer F.Cu) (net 12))
 (segment (start 143.5157 120.7389) (end 142.5702 120.7389) (width 0.4) (layer F.Cu) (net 12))
 (segment (start 141.7766 121.5325) (end 139.7254 121.5325) (width 0.4) (layer F.Cu) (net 12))
 (segment (start 142.5702 120.7389) (end 141.7766 121.5325) (width 0.4) (layer F.Cu) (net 12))
 (segment (start 143.668117 124.562701) (end 144.679501 124.562701) (width 0.4) (layer F.Cu) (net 14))
 (segment (start 138.690818 129.54) (end 143.668117 124.562701) (width 0.4) (layer F.Cu) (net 14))
 (segment (start 137.16 129.54) (end 138.690818 129.54) (width 0.4) (layer F.Cu) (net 14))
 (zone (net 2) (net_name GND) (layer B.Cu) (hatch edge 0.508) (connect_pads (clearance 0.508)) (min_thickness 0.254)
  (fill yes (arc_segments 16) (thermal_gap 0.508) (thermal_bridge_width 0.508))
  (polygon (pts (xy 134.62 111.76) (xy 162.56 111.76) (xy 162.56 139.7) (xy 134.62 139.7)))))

